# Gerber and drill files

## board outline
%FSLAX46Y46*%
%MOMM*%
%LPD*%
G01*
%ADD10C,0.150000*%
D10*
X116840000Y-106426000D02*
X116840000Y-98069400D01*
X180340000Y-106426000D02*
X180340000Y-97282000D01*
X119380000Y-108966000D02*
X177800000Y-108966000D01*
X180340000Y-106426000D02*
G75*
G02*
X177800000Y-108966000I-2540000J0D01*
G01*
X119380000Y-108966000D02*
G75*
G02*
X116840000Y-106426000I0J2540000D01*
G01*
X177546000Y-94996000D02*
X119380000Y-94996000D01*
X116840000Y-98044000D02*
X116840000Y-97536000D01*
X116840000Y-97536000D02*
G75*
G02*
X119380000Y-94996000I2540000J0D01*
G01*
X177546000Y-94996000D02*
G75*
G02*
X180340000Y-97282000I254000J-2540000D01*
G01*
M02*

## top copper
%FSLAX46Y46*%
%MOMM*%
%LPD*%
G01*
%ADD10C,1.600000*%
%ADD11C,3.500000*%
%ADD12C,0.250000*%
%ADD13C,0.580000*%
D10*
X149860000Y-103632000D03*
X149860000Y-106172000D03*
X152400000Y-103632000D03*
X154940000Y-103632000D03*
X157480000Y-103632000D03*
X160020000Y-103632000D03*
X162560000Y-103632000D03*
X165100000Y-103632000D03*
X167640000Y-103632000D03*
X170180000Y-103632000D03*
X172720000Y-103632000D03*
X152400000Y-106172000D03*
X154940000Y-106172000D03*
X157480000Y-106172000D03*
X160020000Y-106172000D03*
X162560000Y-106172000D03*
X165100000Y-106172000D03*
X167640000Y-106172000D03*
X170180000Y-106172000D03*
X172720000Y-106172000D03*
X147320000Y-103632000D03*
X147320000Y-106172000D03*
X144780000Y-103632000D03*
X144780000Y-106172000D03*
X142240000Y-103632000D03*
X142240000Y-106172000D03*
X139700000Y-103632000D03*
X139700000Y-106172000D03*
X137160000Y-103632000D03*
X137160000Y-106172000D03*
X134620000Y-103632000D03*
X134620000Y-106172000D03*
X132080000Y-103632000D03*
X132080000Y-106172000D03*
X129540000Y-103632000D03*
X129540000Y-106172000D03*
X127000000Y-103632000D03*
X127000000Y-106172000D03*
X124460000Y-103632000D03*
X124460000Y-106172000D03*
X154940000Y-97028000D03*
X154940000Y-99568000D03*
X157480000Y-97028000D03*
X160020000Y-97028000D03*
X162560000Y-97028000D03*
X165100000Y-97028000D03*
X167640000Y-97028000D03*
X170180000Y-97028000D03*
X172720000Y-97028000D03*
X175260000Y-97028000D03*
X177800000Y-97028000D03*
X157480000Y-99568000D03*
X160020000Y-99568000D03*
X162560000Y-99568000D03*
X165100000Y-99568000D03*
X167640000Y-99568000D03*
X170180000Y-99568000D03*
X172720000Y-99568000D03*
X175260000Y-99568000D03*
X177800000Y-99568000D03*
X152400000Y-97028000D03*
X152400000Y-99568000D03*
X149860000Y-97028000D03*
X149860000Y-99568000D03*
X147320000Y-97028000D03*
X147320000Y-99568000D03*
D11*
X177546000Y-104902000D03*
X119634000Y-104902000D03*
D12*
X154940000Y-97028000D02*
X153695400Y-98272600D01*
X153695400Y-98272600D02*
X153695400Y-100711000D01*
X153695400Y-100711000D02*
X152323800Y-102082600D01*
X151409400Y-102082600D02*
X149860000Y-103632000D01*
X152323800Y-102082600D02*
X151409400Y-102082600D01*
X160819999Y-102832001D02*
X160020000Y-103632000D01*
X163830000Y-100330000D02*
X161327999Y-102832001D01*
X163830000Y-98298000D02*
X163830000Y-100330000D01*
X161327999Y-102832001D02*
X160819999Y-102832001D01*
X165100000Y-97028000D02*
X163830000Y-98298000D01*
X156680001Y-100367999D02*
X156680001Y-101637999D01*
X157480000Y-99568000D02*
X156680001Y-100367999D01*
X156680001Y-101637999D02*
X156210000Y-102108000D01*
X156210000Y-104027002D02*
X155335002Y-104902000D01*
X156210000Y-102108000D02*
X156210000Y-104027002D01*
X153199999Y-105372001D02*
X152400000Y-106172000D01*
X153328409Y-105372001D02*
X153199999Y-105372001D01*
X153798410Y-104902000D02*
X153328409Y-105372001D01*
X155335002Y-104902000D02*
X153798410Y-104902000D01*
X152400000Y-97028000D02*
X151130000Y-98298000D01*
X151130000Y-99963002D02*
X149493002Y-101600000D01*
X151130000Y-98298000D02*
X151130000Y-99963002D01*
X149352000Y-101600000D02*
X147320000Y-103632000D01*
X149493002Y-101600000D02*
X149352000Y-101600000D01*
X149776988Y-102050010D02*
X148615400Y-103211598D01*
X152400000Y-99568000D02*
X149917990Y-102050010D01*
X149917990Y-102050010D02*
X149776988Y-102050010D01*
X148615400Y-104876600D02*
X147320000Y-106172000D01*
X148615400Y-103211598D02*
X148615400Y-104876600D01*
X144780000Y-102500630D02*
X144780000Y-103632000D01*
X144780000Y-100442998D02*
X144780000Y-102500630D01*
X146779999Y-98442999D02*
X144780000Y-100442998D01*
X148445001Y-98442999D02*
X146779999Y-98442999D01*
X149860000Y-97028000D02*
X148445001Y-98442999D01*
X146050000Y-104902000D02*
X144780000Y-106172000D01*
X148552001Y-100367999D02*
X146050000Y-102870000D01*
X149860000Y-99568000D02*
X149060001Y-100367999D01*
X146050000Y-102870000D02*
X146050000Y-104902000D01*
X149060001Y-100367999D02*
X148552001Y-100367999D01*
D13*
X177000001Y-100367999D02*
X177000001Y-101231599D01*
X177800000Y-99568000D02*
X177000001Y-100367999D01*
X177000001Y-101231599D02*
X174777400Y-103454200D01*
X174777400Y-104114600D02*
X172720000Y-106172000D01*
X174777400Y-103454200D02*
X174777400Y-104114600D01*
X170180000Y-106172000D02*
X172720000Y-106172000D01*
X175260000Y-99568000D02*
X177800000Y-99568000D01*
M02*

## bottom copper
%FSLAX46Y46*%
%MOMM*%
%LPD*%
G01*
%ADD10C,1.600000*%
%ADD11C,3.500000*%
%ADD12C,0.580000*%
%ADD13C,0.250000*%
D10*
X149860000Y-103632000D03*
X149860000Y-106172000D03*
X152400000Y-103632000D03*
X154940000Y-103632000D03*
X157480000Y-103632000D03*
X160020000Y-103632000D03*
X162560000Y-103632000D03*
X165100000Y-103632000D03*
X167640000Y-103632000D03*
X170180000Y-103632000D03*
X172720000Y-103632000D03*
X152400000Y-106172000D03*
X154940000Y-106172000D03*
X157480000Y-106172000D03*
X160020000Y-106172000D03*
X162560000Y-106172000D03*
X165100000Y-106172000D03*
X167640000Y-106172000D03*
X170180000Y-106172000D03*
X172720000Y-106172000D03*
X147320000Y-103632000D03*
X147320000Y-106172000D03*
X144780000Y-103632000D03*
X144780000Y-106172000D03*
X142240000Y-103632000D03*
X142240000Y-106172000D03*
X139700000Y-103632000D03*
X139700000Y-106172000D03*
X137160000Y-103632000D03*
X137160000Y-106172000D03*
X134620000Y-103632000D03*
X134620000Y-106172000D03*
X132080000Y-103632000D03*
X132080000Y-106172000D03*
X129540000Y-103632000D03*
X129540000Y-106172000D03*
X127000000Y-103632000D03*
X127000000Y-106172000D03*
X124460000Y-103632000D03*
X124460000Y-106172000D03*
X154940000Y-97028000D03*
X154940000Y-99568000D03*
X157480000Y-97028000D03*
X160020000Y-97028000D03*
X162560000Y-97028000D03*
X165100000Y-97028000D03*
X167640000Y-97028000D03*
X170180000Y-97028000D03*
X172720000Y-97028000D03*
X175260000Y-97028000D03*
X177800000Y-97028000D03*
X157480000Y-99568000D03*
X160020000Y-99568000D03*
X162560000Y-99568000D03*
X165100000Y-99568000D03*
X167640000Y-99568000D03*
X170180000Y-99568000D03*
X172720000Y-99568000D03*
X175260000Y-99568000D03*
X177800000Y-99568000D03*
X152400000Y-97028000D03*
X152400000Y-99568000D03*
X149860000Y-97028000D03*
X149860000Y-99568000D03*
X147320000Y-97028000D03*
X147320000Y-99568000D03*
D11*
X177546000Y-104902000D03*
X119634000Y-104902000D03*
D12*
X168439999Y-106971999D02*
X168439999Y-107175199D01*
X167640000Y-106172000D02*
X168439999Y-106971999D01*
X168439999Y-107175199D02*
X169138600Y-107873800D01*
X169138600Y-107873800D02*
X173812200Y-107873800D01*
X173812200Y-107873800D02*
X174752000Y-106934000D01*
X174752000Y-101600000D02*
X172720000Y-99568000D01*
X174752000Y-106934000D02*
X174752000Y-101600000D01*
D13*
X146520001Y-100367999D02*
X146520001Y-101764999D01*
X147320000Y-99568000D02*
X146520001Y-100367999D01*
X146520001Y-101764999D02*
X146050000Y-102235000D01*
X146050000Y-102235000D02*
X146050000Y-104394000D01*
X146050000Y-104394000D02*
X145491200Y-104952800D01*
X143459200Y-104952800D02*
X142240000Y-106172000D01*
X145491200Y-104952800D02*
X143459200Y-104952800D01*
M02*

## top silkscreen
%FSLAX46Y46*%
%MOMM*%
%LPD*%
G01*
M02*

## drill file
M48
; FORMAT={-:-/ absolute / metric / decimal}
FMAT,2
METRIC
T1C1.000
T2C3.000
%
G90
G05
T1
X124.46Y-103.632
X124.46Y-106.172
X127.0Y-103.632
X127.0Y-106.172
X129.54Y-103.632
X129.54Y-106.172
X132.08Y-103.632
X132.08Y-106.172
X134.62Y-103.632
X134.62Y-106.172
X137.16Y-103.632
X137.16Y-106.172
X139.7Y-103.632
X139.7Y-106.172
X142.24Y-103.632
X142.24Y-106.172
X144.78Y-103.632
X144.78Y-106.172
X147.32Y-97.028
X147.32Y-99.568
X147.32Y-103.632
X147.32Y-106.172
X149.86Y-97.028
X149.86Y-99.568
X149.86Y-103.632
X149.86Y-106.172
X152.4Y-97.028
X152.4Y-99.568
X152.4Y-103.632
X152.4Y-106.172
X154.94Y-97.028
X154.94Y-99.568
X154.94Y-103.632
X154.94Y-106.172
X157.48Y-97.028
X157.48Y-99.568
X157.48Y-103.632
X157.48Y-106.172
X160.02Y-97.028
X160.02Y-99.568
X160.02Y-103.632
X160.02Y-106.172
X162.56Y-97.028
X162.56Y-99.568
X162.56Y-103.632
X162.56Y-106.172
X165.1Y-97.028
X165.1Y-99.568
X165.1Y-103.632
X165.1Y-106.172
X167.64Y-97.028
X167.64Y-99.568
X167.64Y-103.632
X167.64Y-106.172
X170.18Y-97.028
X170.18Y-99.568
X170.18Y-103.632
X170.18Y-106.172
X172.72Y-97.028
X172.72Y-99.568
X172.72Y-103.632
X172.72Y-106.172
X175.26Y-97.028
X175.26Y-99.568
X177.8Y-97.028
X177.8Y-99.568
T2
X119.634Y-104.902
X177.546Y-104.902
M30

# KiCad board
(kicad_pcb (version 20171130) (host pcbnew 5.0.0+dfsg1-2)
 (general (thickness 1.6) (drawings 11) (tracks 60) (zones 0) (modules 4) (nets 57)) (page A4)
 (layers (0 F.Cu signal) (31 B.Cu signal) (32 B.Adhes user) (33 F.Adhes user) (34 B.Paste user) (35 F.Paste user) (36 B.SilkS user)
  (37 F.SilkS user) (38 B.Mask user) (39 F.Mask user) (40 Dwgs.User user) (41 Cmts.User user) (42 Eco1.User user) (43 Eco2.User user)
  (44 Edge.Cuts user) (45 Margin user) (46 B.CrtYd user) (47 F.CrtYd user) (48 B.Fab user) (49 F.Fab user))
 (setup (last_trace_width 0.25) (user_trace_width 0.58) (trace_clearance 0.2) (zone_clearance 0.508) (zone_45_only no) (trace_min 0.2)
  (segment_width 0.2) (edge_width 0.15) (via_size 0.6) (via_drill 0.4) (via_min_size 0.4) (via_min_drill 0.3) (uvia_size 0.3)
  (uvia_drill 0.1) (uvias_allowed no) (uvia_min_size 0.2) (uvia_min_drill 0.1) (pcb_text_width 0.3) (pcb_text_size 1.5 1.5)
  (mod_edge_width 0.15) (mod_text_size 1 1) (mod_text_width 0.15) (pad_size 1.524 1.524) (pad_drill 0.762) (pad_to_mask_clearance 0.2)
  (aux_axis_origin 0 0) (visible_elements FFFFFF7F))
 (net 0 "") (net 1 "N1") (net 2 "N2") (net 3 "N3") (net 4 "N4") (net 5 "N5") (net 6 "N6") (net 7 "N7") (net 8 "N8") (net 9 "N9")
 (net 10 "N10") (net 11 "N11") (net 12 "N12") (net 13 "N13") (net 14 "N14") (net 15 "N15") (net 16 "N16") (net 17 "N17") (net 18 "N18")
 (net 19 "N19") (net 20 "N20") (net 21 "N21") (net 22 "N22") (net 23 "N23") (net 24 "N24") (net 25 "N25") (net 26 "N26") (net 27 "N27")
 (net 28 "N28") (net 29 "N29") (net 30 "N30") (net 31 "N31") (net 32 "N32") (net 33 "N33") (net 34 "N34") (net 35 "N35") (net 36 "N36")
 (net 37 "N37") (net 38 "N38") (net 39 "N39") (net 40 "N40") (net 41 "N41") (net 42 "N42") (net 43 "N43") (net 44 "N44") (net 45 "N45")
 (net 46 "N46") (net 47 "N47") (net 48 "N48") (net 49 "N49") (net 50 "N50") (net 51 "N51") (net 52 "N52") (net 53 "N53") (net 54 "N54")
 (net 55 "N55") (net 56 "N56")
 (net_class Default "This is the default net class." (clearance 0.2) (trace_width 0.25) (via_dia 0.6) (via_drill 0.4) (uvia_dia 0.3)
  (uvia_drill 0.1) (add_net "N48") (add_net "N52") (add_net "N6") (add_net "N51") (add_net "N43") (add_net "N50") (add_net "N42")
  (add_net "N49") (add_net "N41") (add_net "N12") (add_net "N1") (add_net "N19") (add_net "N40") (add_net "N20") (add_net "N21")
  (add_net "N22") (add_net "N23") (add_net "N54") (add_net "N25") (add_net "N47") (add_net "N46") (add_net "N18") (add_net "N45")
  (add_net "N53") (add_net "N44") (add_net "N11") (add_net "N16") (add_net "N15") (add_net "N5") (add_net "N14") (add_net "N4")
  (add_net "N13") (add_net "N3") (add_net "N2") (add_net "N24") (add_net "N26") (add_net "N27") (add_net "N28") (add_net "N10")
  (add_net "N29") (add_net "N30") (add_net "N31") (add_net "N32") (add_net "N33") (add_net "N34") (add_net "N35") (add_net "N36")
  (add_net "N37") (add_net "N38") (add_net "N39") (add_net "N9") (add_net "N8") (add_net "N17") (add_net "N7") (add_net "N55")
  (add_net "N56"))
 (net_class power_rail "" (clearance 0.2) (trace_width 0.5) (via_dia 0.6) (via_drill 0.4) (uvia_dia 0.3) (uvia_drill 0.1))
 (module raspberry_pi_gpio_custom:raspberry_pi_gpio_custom (layer F.Cu) (at 148.59 104.902)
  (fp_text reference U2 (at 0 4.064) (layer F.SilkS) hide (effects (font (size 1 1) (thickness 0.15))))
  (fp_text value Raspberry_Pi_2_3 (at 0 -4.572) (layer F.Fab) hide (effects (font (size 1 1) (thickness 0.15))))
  (pad 19 thru_hole circle (at 1.27 -1.27) (size 1.6 1.6) (drill 1) (layers *.Cu *.Mask) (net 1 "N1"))
  (pad 20 thru_hole circle (at 1.27 1.27) (size 1.6 1.6) (drill 1) (layers *.Cu *.Mask) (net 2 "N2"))
  (pad 17 thru_hole circle (at 3.81 -1.27) (size 1.6 1.6) (drill 1) (layers *.Cu *.Mask) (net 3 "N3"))
  (pad 15 thru_hole circle (at 6.35 -1.27) (size 1.6 1.6) (drill 1) (layers *.Cu *.Mask) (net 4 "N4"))
  (pad 13 thru_hole circle (at 8.89 -1.27) (size 1.6 1.6) (drill 1) (layers *.Cu *.Mask) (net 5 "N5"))
  (pad 11 thru_hole circle (at 11.43 -1.27) (size 1.6 1.6) (drill 1) (layers *.Cu *.Mask) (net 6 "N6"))
  (pad 9 thru_hole circle (at 13.97 -1.27) (size 1.6 1.6) (drill 1) (layers *.Cu *.Mask) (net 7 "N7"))
  (pad 7 thru_hole circle (at 16.51 -1.27) (size 1.6 1.6) (drill 1) (layers *.Cu *.Mask) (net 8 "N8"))
  (pad 5 thru_hole circle (at 19.05 -1.27) (size 1.6 1.6) (drill 1) (layers *.Cu *.Mask) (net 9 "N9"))
  (pad 3 thru_hole circle (at 21.59 -1.27) (size 1.6 1.6) (drill 1) (layers *.Cu *.Mask) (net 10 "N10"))
  (pad 1 thru_hole circle (at 24.13 -1.27) (size 1.6 1.6) (drill 1) (layers *.Cu *.Mask) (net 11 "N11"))
  (pad 18 thru_hole circle (at 3.81 1.27) (size 1.6 1.6) (drill 1) (layers *.Cu *.Mask) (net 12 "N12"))
  (pad 16 thru_hole circle (at 6.35 1.27) (size 1.6 1.6) (drill 1) (layers *.Cu *.Mask) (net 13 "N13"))
  (pad 14 thru_hole circle (at 8.89 1.27) (size 1.6 1.6) (drill 1) (layers *.Cu *.Mask) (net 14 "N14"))
  (pad 12 thru_hole circle (at 11.43 1.27) (size 1.6 1.6) (drill 1) (layers *.Cu *.Mask) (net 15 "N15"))
  (pad 10 thru_hole circle (at 13.97 1.27) (size 1.6 1.6) (drill 1) (layers *.Cu *.Mask) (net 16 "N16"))
  (pad 8 thru_hole circle (at 16.51 1.27) (size 1.6 1.6) (drill 1) (layers *.Cu *.Mask) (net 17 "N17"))
  (pad 6 thru_hole circle (at 19.05 1.27) (size 1.6 1.6) (drill 1) (layers *.Cu *.Mask) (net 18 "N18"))
  (pad 4 thru_hole circle (at 21.59 1.27) (size 1.6 1.6) (drill 1) (layers *.Cu *.Mask) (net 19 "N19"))
  (pad 2 thru_hole circle (at 24.13 1.27) (size 1.6 1.6) (drill 1) (layers *.Cu *.Mask) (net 19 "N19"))
  (pad 21 thru_hole circle (at -1.27 -1.27) (size 1.6 1.6) (drill 1) (layers *.Cu *.Mask) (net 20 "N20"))
  (pad 22 thru_hole circle (at -1.27 1.27) (size 1.6 1.6) (drill 1) (layers *.Cu *.Mask) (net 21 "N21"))
  (pad 23 thru_hole circle (at -3.81 -1.27) (size 1.6 1.6) (drill 1) (layers *.Cu *.Mask) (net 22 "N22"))
  (pad 24 thru_hole circle (at -3.81 1.27) (size 1.6 1.6) (drill 1) (layers *.Cu *.Mask) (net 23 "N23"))
  (pad 25 thru_hole circle (at -6.35 -1.27) (size 1.6 1.6) (drill 1) (layers *.Cu *.Mask) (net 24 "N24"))
  (pad 26 thru_hole circle (at -6.35 1.27) (size 1.6 1.6) (drill 1) (layers *.Cu *.Mask) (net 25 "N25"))
  (pad 27 thru_hole circle (at -8.89 -1.27) (size 1.6 1.6) (drill 1) (layers *.Cu *.Mask) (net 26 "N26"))
  (pad 28 thru_hole circle (at -8.89 1.27) (size 1.6 1.6) (drill 1) (layers *.Cu *.Mask) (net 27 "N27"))
  (pad 29 thru_hole circle (at -11.43 -1.27) (size 1.6 1.6) (drill 1) (layers *.Cu *.Mask) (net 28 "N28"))
  (pad 30 thru_hole circle (at -11.43 1.27) (size 1.6 1.6) (drill 1) (layers *.Cu *.Mask) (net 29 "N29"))
  (pad 31 thru_hole circle (at -13.97 -1.27) (size 1.6 1.6) (drill 1) (layers *.Cu *.Mask) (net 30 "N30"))
  (pad 32 thru_hole circle (at -13.97 1.27) (size 1.6 1.6) (drill 1) (layers *.Cu *.Mask) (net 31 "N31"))
  (pad 33 thru_hole circle (at -16.51 -1.27) (size 1.6 1.6) (drill 1) (layers *.Cu *.Mask) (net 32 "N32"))
  (pad 34 thru_hole circle (at -16.51 1.27) (size 1.6 1.6) (drill 1) (layers *.Cu *.Mask) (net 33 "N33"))
  (pad 35 thru_hole circle (at -19.05 -1.27) (size 1.6 1.6) (drill 1) (layers *.Cu *.Mask) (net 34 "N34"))
  (pad 36 thru_hole circle (at -19.05 1.27) (size 1.6 1.6) (drill 1) (layers *.Cu *.Mask) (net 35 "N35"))
  (pad 37 thru_hole circle (at -21.59 -1.27) (size 1.6 1.6) (drill 1) (layers *.Cu *.Mask) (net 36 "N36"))
  (pad 38 thru_hole circle (at -21.59 1.27) (size 1.6 1.6) (drill 1) (layers *.Cu *.Mask) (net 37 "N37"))
  (pad 39 thru_hole circle (at -24.13 -1.27) (size 1.6 1.6) (drill 1) (layers *.Cu *.Mask) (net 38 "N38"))
  (pad 40 thru_hole circle (at -24.13 1.27) (size 1.6 1.6) (drill 1) (layers *.Cu *.Mask) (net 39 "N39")))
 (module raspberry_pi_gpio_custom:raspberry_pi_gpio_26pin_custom (layer F.Cu) (at 162.56 98.298)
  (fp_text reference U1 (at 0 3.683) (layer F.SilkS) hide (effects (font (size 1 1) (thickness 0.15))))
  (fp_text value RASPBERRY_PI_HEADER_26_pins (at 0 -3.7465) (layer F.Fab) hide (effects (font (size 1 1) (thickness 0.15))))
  (pad 19 thru_hole circle (at -7.62 -1.27) (size 1.6 1.6) (drill 1) (layers *.Cu *.Mask) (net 1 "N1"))
  (pad 20 thru_hole circle (at -7.62 1.27) (size 1.6 1.6) (drill 1) (layers *.Cu *.Mask) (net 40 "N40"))
  (pad 17 thru_hole circle (at -5.08 -1.27) (size 1.6 1.6) (drill 1) (layers *.Cu *.Mask) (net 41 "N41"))
  (pad 15 thru_hole circle (at -2.54 -1.27) (size 1.6 1.6) (drill 1) (layers *.Cu *.Mask) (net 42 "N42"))
  (pad 13 thru_hole circle (at 0 -1.27) (size 1.6 1.6) (drill 1) (layers *.Cu *.Mask) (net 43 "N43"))
  (pad 11 thru_hole circle (at 2.54 -1.27) (size 1.6 1.6) (drill 1) (layers *.Cu *.Mask) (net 6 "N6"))
  (pad 9 thru_hole circle (at 5.08 -1.27) (size 1.6 1.6) (drill 1) (layers *.Cu *.Mask) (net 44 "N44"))
  (pad 7 thru_hole circle (at 7.62 -1.27) (size 1.6 1.6) (drill 1) (layers *.Cu *.Mask) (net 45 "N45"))
  (pad 5 thru_hole circle (at 10.16 -1.27) (size 1.6 1.6) (drill 1) (layers *.Cu *.Mask) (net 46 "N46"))
  (pad 3 thru_hole circle (at 12.7 -1.27) (size 1.6 1.6) (drill 1) (layers *.Cu *.Mask) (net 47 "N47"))
  (pad 1 thru_hole circle (at 15.24 -1.27) (size 1.6 1.6) (drill 1) (layers *.Cu *.Mask) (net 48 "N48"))
  (pad 18 thru_hole circle (at -5.08 1.27) (size 1.6 1.6) (drill 1) (layers *.Cu *.Mask) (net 12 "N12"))
  (pad 16 thru_hole circle (at -2.54 1.27) (size 1.6 1.6) (drill 1) (layers *.Cu *.Mask) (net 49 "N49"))
  (pad 14 thru_hole circle (at 0 1.27) (size 1.6 1.6) (drill 1) (layers *.Cu *.Mask) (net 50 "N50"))
  (pad 12 thru_hole circle (at 2.54 1.27) (size 1.6 1.6) (drill 1) (layers *.Cu *.Mask) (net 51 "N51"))
  (pad 10 thru_hole circle (at 5.08 1.27) (size 1.6 1.6) (drill 1) (layers *.Cu *.Mask) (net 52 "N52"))
  (pad 8 thru_hole circle (at 7.62 1.27) (size 1.6 1.6) (drill 1) (layers *.Cu *.Mask) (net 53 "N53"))
  (pad 6 thru_hole circle (at 10.16 1.27) (size 1.6 1.6) (drill 1) (layers *.Cu *.Mask) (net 18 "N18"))
  (pad 4 thru_hole circle (at 12.7 1.27) (size 1.6 1.6) (drill 1) (layers *.Cu *.Mask) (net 19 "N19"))
  (pad 2 thru_hole circle (at 15.24 1.27) (size 1.6 1.6) (drill 1) (layers *.Cu *.Mask) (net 19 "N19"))
  (pad 21 thru_hole circle (at -10.16 -1.27) (size 1.6 1.6) (drill 1) (layers *.Cu *.Mask) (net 20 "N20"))
  (pad 22 thru_hole circle (at -10.16 1.27) (size 1.6 1.6) (drill 1) (layers *.Cu *.Mask) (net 21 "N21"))
  (pad 23 thru_hole circle (at -12.7 -1.27) (size 1.6 1.6) (drill 1) (layers *.Cu *.Mask) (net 22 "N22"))
  (pad 24 thru_hole circle (at -12.7 1.27) (size 1.6 1.6) (drill 1) (layers *.Cu *.Mask) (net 23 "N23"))
  (pad 25 thru_hole circle (at -15.24 -1.27) (size 1.6 1.6) (drill 1) (layers *.Cu *.Mask) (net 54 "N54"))
  (pad 26 thru_hole circle (at -15.24 1.27) (size 1.6 1.6) (drill 1) (layers *.Cu *.Mask) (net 25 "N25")))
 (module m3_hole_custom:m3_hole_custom (layer F.Cu) (at 177.546 104.902)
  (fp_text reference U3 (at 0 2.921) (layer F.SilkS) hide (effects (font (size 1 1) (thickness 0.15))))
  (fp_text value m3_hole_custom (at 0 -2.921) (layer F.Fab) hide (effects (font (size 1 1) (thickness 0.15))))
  (pad 1 thru_hole circle (at 0 0) (size 3.5 3.5) (drill 3) (layers *.Cu *.Mask) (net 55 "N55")))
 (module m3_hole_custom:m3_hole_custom (layer F.Cu) (at 119.634 104.902)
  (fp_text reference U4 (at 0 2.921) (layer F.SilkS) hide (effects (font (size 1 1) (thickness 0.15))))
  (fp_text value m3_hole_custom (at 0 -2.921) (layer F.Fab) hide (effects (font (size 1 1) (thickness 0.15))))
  (pad 1 thru_hole circle (at 0 0) (size 3.5 3.5) (drill 3) (layers *.Cu *.Mask) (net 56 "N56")))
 (gr_line (start 116.84 106.426) (end 116.84 98.0694) (layer Edge.Cuts) (width 0.15))
 (gr_line (start 180.34 106.426) (end 180.34 97.282) (layer Edge.Cuts) (width 0.15))
 (gr_line (start 119.38 108.966) (end 177.8 108.966) (layer Edge.Cuts) (width 0.15))
 (gr_arc (start 177.8 106.426) (end 177.8 108.966) (angle -90) (layer Edge.Cuts) (width 0.15))
 (gr_arc (start 119.38 106.426) (end 116.84 106.426) (angle -90) (layer Edge.Cuts) (width 0.15))
 (gr_line (start 177.546 94.996) (end 119.38 94.996) (angle 90) (layer Edge.Cuts) (width 0.15))
 (gr_line (start 116.84 98.044) (end 116.84 97.536) (angle 90) (layer Edge.Cuts) (width 0.15))
 (gr_arc (start 119.38 97.536) (end 116.84 97.536) (angle 90) (layer Edge.Cuts) (width 0.15))
 (gr_arc (start 177.8 97.536) (end 177.546 94.996) (angle 90) (layer Edge.Cuts) (width 0.15))
 (segment (start 154.94 97.028) (end 153.6954 98.2726) (width 0.25) (layer F.Cu) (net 1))
 (segment (start 153.6954 98.2726) (end 153.6954 100.711) (width 0.25) (layer F.Cu) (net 1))
 (segment (start 153.6954 100.711) (end 152.3238 102.0826) (width 0.25) (layer F.Cu) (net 1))
 (segment (start 151.4094 102.0826) (end 149.86 103.632) (width 0.25) (layer F.Cu) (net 1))
 (segment (start 152.3238 102.0826) (end 151.4094 102.0826) (width 0.25) (layer F.Cu) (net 1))
 (segment (start 160.819999 102.832001) (end 160.02 103.632) (width 0.25) (layer F.Cu) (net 6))
 (segment (start 163.83 100.33) (end 161.327999 102.832001) (width 0.25) (layer F.Cu) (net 6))
 (segment (start 163.83 98.298) (end 163.83 100.33) (width 0.25) (layer F.Cu) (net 6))
 (segment (start 161.327999 102.832001) (end 160.819999 102.832001) (width 0.25) (layer F.Cu) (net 6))
 (segment (start 165.1 97.028) (end 163.83 98.298) (width 0.25) (layer F.Cu) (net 6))
 (segment (start 156.680001 100.367999) (end 156.680001 101.637999) (width 0.25) (layer F.Cu) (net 12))
 (segment (start 157.48 99.568) (end 156.680001 100.367999) (width 0.25) (layer F.Cu) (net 12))
 (segment (start 156.680001 101.637999) (end 156.21 102.108) (width 0.25) (layer F.Cu) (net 12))
 (segment (start 156.21 104.027002) (end 155.335002 104.902) (width 0.25) (layer F.Cu) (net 12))
 (segment (start 156.21 102.108) (end 156.21 104.027002) (width 0.25) (layer F.Cu) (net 12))
 (segment (start 153.199999 105.372001) (end 152.4 106.172) (width 0.25) (layer F.Cu) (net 12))
 (segment (start 153.328409 105.372001) (end 153.199999 105.372001) (width 0.25) (layer F.Cu) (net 12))
 (segment (start 153.79841 104.902) (end 153.328409 105.372001) (width 0.25) (layer F.Cu) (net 12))
 (segment (start 155.335002 104.902) (end 153.79841 104.902) (width 0.25) (layer F.Cu) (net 12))
 (segment (start 168.439999 106.971999) (end 168.439999 107.175199) (width 0.58) (layer B.Cu) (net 18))
 (segment (start 167.64 106.172) (end 168.439999 106.971999) (width 0.58) (layer B.Cu) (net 18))
 (segment (start 168.439999 107.175199) (end 169.1386 107.8738) (width 0.58) (layer B.Cu) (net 18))
 (segment (start 169.1386 107.8738) (end 173.8122 107.8738) (width 0.58) (layer B.Cu) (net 18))
 (segment (start 173.8122 107.8738) (end 174.752 106.934) (width 0.58) (layer B.Cu) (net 18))
 (segment (start 174.752 101.6) (end 172.72 99.568) (width 0.58) (layer B.Cu) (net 18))
 (segment (start 174.752 106.934) (end 174.752 101.6) (width 0.58) (layer B.Cu) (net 18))
 (segment (start 152.4 97.028) (end 151.13 98.298) (width 0.25) (layer F.Cu) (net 20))
 (segment (start 151.13 99.963002) (end 149.493002 101.6) (width 0.25) (layer F.Cu) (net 20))
 (segment (start 151.13 98.298) (end 151.13 99.963002) (width 0.25) (layer F.Cu) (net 20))
 (segment (start 149.352 101.6) (end 147.32 103.632) (width 0.25) (layer F.Cu) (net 20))
 (segment (start 149.493002 101.6) (end 149.352 101.6) (width 0.25) (layer F.Cu) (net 20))
 (segment (start 149.776988 102.05001) (end 148.6154 103.211598) (width 0.25) (layer F.Cu) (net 21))
 (segment (start 152.4 99.568) (end 149.91799 102.05001) (width 0.25) (layer F.Cu) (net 21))
 (segment (start 149.91799 102.05001) (end 149.776988 102.05001) (width 0.25) (layer F.Cu) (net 21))
 (segment (start 148.6154 104.8766) (end 147.32 106.172) (width 0.25) (layer F.Cu) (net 21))
 (segment (start 148.6154 103.211598) (end 148.6154 104.8766) (width 0.25) (layer F.Cu) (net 21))
 (segment (start 144.78 102.50063) (end 144.78 103.632) (width 0.25) (layer F.Cu) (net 22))
 (segment (start 144.78 100.442998) (end 144.78 102.50063) (width 0.25) (layer F.Cu) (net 22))
 (segment (start 146.779999 98.442999) (end 144.78 100.442998) (width 0.25) (layer F.Cu) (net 22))
 (segment (start 148.445001 98.442999) (end 146.779999 98.442999) (width 0.25) (layer F.Cu) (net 22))
 (segment (start 149.86 97.028) (end 148.445001 98.442999) (width 0.25) (layer F.Cu) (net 22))
 (segment (start 146.05 104.902) (end 144.78 106.172) (width 0.25) (layer F.Cu) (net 23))
 (segment (start 148.552001 100.367999) (end 146.05 102.87) (width 0.25) (layer F.Cu) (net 23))
 (segment (start 149.86 99.568) (end 149.060001 100.367999) (width 0.25) (layer F.Cu) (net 23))
 (segment (start 146.05 102.87) (end 146.05 104.902) (width 0.25) (layer F.Cu) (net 23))
 (segment (start 149.060001 100.367999) (end 148.552001 100.367999) (width 0.25) (layer F.Cu) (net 23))
 (segment (start 146.520001 100.367999) (end 146.520001 101.764999) (width 0.25) (layer B.Cu) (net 25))
 (segment (start 147.32 99.568) (end 146.520001 100.367999) (width 0.25) (layer B.Cu) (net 25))
 (segment (start 146.520001 101.764999) (end 146.05 102.235) (width 0.25) (layer B.Cu) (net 25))
 (segment (start 146.05 102.235) (end 146.05 104.394) (width 0.25) (layer B.Cu) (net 25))
 (segment (start 146.05 104.394) (end 145.4912 104.9528) (width 0.25) (layer B.Cu) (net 25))
 (segment (start 143.4592 104.9528) (end 142.24 106.172) (width 0.25) (layer B.Cu) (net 25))
 (segment (start 145.4912 104.9528) (end 143.4592 104.9528) (width 0.25) (layer B.Cu) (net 25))
 (segment (start 177.000001 100.367999) (end 177.000001 101.231599) (width 0.58) (layer F.Cu) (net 19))
 (segment (start 177.8 99.568) (end 177.000001 100.367999) (width 0.58) (layer F.Cu) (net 19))
 (segment (start 177.000001 101.231599) (end 174.7774 103.4542) (width 0.58) (layer F.Cu) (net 19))
 (segment (start 174.7774 104.1146) (end 172.72 106.172) (width 0.58) (layer F.Cu) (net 19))
 (segment (start 174.7774 103.4542) (end 174.7774 104.1146) (width 0.58) (layer F.Cu) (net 19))
 (segment (start 170.18 106.172) (end 172.72 106.172) (width 0.58) (layer F.Cu) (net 19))
 (segment (start 175.26 99.568) (end 177.8 99.568) (width 0.58) (layer F.Cu) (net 19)))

